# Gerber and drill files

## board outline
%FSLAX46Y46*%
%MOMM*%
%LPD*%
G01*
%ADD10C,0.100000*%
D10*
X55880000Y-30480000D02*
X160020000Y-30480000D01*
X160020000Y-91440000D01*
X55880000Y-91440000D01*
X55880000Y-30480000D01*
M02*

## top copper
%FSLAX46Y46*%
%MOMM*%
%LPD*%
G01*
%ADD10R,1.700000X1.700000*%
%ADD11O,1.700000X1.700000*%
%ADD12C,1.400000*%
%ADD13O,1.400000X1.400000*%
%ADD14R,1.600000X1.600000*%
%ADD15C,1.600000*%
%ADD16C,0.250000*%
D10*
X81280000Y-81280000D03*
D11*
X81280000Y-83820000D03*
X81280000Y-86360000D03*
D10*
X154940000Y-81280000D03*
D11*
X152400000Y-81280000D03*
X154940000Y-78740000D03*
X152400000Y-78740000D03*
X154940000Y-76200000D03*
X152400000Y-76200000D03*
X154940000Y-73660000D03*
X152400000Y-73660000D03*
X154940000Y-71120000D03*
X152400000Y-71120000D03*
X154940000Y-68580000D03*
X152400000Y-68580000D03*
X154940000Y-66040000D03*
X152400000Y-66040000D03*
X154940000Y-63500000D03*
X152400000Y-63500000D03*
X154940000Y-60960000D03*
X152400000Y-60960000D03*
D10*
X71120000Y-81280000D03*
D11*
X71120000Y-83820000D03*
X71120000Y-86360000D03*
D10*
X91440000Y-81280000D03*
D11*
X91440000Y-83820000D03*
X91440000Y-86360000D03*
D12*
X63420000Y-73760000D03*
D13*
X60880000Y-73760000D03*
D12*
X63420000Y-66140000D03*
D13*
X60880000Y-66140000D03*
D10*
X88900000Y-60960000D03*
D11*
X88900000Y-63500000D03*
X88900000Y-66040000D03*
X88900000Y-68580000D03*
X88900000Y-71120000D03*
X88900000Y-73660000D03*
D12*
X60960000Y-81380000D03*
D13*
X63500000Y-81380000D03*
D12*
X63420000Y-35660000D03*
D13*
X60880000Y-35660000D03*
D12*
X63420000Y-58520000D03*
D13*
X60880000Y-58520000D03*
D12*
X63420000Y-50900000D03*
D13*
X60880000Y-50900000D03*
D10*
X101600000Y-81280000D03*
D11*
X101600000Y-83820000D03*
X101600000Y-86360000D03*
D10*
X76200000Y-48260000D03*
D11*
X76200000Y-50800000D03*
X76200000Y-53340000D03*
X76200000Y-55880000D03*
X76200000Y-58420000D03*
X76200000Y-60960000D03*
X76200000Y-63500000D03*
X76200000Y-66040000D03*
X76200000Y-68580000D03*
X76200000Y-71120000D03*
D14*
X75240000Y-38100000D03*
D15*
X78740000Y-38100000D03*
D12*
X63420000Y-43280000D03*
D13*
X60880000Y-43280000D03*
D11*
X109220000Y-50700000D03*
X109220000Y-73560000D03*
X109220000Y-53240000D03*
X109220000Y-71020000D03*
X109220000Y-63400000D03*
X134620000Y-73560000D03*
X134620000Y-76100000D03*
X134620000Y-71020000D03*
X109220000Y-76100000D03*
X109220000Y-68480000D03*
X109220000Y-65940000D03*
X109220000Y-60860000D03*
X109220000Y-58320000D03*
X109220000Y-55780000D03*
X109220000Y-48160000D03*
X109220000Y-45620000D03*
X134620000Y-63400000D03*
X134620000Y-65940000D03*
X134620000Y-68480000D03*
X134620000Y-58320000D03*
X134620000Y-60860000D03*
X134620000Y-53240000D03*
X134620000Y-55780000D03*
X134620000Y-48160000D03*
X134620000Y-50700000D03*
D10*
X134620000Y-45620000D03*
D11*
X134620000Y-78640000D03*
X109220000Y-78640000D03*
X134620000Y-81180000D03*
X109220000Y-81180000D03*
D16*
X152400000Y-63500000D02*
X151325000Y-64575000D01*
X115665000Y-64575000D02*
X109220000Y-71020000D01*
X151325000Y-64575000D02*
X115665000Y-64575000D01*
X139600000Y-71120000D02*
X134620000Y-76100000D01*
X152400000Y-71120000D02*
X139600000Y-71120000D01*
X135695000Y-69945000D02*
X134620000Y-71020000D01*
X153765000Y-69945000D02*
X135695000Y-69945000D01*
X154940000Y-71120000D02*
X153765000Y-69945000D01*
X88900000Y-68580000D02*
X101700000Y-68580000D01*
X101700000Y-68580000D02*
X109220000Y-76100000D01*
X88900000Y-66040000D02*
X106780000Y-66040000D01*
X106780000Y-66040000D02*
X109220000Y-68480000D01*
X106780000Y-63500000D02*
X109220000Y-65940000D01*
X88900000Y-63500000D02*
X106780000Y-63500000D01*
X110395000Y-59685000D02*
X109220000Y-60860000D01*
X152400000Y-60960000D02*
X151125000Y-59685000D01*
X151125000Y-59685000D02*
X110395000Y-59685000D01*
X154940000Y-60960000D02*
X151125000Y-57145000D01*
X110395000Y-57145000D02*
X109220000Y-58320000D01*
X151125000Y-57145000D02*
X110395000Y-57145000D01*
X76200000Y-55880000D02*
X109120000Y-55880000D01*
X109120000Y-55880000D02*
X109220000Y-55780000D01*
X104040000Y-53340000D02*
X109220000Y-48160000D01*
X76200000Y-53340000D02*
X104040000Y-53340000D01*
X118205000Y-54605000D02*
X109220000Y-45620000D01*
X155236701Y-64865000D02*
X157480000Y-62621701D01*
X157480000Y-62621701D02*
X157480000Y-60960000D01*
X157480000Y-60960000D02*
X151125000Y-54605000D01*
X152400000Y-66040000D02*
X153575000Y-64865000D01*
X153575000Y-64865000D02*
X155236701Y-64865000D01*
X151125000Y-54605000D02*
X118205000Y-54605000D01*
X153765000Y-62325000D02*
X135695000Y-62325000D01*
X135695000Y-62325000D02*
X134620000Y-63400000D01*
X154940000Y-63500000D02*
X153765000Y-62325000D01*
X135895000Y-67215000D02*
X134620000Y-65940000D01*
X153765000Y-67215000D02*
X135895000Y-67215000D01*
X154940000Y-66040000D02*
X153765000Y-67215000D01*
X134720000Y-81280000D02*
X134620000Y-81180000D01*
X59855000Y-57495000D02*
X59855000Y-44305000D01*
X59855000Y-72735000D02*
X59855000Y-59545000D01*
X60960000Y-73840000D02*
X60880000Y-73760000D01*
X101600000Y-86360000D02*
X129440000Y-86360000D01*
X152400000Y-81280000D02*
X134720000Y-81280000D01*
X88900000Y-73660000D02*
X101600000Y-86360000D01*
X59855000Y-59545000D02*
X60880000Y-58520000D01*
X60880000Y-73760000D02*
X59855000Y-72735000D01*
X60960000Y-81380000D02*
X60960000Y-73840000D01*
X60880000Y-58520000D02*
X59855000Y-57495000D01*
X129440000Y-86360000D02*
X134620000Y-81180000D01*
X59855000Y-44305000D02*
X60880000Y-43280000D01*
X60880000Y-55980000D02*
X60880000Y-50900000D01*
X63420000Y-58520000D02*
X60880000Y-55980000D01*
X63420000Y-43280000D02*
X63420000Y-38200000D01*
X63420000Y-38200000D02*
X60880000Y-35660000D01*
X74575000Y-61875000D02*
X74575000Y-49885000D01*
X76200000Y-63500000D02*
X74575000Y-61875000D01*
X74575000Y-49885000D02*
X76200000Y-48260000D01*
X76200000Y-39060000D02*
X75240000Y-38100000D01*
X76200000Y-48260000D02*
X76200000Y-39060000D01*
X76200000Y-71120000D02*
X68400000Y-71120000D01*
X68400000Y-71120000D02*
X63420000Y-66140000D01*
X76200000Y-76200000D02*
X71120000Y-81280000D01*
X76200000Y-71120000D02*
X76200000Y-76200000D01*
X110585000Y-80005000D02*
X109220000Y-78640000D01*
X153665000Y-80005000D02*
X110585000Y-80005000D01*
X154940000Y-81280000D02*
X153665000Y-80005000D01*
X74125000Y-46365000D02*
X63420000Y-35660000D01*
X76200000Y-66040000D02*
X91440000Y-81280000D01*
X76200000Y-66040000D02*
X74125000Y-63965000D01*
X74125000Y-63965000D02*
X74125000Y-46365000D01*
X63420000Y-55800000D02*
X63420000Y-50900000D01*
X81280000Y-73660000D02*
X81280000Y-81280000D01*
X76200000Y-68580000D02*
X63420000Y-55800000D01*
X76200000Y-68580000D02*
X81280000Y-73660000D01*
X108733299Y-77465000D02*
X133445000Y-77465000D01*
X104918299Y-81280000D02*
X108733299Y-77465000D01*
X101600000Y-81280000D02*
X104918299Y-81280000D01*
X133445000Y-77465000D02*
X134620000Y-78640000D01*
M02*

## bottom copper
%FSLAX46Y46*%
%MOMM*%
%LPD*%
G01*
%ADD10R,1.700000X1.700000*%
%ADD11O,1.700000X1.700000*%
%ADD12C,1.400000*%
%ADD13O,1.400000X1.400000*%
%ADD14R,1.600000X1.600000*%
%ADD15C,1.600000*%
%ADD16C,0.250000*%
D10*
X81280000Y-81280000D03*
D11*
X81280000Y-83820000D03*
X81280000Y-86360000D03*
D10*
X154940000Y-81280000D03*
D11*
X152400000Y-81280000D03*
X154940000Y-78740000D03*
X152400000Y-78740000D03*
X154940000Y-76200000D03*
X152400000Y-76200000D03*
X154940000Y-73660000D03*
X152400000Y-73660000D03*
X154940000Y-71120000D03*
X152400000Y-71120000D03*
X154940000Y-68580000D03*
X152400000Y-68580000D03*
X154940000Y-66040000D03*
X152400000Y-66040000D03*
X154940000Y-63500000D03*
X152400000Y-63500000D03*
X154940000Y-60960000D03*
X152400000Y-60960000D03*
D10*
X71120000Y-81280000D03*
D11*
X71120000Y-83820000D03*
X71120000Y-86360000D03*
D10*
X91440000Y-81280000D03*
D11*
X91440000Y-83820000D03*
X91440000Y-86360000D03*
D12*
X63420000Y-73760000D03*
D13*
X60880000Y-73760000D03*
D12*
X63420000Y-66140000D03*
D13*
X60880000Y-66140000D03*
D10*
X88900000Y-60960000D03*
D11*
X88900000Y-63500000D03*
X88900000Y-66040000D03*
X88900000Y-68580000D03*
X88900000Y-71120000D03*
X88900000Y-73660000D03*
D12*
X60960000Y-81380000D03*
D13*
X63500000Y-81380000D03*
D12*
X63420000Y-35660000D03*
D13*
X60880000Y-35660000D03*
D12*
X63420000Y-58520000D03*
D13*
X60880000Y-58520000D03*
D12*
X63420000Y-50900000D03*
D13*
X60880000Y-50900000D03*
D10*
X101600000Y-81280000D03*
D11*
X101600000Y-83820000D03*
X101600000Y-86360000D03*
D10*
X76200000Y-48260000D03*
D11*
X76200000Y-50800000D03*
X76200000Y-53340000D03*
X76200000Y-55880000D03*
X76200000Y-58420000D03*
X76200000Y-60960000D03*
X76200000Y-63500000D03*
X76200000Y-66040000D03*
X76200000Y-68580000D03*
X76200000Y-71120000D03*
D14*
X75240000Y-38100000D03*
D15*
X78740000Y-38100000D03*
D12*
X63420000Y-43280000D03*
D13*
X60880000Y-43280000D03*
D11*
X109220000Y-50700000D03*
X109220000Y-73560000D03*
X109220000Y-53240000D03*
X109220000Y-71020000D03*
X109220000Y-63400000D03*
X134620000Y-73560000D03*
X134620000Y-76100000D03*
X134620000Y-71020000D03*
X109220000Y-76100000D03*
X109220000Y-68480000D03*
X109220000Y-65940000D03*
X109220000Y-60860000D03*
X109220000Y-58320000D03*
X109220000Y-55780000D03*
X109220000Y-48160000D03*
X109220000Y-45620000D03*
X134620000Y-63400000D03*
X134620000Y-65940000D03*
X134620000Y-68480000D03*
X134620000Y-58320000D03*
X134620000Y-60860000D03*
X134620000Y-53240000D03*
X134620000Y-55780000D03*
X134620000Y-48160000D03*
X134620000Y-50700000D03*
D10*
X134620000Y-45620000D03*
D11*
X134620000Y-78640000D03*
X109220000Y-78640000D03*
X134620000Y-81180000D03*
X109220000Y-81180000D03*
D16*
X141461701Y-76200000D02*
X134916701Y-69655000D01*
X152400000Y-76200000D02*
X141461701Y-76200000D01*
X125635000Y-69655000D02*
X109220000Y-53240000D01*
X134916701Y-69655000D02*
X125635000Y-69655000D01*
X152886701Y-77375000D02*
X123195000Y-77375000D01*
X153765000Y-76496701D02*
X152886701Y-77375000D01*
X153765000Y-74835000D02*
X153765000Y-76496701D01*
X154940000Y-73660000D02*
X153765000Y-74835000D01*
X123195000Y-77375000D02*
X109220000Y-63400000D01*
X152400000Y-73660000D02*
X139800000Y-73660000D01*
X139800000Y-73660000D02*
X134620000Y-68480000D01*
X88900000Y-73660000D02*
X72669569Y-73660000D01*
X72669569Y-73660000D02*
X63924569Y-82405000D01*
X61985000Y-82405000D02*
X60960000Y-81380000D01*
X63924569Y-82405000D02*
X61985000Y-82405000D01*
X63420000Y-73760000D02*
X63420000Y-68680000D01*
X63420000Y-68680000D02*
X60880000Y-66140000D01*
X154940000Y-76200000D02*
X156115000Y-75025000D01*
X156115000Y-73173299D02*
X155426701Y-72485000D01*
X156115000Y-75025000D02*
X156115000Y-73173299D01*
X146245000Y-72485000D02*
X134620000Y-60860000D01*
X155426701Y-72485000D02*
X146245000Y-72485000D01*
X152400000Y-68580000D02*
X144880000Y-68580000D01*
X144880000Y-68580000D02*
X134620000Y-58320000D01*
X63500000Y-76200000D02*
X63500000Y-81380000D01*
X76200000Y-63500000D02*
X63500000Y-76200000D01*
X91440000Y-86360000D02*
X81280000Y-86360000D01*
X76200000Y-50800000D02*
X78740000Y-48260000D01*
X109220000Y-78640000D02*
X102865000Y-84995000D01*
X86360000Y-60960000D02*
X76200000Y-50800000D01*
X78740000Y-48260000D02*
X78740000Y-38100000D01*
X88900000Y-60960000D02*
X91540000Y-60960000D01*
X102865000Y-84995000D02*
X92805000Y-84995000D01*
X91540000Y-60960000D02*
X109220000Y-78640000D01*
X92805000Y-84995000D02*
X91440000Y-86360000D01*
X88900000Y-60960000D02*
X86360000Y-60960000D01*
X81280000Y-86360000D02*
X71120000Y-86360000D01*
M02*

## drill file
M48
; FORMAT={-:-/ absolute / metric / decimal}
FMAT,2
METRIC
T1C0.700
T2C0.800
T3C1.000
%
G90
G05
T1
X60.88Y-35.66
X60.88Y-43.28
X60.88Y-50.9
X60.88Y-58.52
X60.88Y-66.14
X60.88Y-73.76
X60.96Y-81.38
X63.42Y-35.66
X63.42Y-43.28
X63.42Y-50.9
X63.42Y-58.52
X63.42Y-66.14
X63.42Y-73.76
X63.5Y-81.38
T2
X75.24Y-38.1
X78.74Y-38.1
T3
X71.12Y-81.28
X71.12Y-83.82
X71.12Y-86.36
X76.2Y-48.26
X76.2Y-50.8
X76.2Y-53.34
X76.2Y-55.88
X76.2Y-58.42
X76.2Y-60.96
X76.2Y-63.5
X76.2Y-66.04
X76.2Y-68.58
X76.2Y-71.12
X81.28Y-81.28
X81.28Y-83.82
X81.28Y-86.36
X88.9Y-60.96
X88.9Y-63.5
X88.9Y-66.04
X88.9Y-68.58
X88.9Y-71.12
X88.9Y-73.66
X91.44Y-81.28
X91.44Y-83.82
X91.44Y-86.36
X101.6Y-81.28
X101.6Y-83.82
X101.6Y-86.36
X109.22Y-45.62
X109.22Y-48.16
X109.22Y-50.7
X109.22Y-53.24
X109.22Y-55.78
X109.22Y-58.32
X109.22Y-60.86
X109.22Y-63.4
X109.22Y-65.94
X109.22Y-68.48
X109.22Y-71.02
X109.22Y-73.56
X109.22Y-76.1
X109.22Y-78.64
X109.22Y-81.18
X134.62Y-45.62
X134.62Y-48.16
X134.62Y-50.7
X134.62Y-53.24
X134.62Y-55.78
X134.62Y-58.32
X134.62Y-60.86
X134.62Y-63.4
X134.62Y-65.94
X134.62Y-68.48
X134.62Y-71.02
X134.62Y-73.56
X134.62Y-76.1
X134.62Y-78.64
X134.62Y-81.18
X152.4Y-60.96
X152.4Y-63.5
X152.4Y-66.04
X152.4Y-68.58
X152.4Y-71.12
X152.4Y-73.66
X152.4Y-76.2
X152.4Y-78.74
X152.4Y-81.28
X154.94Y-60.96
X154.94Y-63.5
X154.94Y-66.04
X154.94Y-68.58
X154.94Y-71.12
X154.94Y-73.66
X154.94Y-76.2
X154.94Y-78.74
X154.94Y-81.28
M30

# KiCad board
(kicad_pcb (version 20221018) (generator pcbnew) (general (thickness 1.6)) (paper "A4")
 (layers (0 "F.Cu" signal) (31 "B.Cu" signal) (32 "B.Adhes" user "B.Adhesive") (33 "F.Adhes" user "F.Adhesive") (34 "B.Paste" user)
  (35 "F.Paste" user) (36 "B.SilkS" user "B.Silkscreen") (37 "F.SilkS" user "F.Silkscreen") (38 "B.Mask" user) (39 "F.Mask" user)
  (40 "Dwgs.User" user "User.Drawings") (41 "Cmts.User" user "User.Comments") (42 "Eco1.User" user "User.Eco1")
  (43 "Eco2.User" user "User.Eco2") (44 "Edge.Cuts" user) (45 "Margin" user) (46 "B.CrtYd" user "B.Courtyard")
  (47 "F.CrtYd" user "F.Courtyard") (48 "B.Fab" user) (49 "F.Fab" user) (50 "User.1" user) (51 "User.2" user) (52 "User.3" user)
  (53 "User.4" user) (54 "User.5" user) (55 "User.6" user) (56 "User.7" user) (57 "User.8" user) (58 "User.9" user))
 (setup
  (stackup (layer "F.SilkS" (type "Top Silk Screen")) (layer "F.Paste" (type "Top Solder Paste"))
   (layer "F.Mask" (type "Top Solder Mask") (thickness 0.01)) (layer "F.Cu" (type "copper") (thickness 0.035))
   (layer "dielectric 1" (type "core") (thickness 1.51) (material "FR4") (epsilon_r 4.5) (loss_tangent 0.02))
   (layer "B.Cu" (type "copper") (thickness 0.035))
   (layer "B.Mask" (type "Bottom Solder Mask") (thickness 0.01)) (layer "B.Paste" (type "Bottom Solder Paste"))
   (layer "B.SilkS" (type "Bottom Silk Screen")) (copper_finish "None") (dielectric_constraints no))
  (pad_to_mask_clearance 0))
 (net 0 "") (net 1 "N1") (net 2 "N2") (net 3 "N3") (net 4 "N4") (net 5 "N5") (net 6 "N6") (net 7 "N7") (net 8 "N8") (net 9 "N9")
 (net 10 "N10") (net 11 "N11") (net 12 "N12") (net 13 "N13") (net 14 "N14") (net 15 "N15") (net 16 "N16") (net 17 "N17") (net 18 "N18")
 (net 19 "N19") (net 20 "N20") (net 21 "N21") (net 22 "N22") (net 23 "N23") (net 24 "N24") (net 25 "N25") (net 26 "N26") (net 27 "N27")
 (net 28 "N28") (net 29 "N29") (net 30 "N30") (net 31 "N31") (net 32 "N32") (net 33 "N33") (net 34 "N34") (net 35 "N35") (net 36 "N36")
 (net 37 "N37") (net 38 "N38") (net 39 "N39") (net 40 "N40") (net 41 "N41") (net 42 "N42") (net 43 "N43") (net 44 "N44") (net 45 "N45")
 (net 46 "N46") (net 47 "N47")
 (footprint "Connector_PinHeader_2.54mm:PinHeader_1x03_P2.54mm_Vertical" (layer "F.Cu") (at 81.28 81.28)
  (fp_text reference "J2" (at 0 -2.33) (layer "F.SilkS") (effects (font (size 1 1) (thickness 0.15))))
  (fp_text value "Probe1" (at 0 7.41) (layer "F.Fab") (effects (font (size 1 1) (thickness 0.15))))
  (pad "1" thru_hole rect (at 0 0) (size 1.7 1.7) (drill 1) (layers "*.Cu" "*.Mask") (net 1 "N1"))
  (pad "2" thru_hole oval (at 0 2.54) (size 1.7 1.7) (drill 1) (layers "*.Cu" "*.Mask") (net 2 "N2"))
  (pad "3" thru_hole oval (at 0 5.08) (size 1.7 1.7) (drill 1) (layers "*.Cu" "*.Mask") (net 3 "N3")))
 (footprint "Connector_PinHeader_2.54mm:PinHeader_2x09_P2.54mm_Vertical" (layer "F.Cu") (at 154.94 81.28 180)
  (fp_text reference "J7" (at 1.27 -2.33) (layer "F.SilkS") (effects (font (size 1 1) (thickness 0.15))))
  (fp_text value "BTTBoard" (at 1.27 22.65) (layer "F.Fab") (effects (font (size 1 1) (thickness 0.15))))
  (pad "1" thru_hole rect (at 0 0 180) (size 1.7 1.7) (drill 1) (layers "*.Cu" "*.Mask") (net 3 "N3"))
  (pad "2" thru_hole oval (at 2.54 0 180) (size 1.7 1.7) (drill 1) (layers "*.Cu" "*.Mask") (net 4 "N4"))
  (pad "3" thru_hole oval (at 0 2.54 180) (size 1.7 1.7) (drill 1) (layers "*.Cu" "*.Mask") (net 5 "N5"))
  (pad "4" thru_hole oval (at 2.54 2.54 180) (size 1.7 1.7) (drill 1) (layers "*.Cu" "*.Mask") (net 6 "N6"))
  (pad "5" thru_hole oval (at 0 5.08 180) (size 1.7 1.7) (drill 1) (layers "*.Cu" "*.Mask") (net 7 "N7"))
  (pad "6" thru_hole oval (at 2.54 5.08 180) (size 1.7 1.7) (drill 1) (layers "*.Cu" "*.Mask") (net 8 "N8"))
  (pad "7" thru_hole oval (at 0 7.62 180) (size 1.7 1.7) (drill 1) (layers "*.Cu" "*.Mask") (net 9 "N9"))
  (pad "8" thru_hole oval (at 2.54 7.62 180) (size 1.7 1.7) (drill 1) (layers "*.Cu" "*.Mask") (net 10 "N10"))
  (pad "9" thru_hole oval (at 0 10.16 180) (size 1.7 1.7) (drill 1) (layers "*.Cu" "*.Mask") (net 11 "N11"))
  (pad "10" thru_hole oval (at 2.54 10.16 180) (size 1.7 1.7) (drill 1) (layers "*.Cu" "*.Mask") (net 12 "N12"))
  (pad "11" thru_hole oval (at 0 12.7 180) (size 1.7 1.7) (drill 1) (layers "*.Cu" "*.Mask") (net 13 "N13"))
  (pad "12" thru_hole oval (at 2.54 12.7 180) (size 1.7 1.7) (drill 1) (layers "*.Cu" "*.Mask") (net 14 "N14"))
  (pad "13" thru_hole oval (at 0 15.24 180) (size 1.7 1.7) (drill 1) (layers "*.Cu" "*.Mask") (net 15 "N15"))
  (pad "14" thru_hole oval (at 2.54 15.24 180) (size 1.7 1.7) (drill 1) (layers "*.Cu" "*.Mask") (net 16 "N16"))
  (pad "15" thru_hole oval (at 0 17.78 180) (size 1.7 1.7) (drill 1) (layers "*.Cu" "*.Mask") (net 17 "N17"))
  (pad "16" thru_hole oval (at 2.54 17.78 180) (size 1.7 1.7) (drill 1) (layers "*.Cu" "*.Mask") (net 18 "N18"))
  (pad "17" thru_hole oval (at 0 20.32 180) (size 1.7 1.7) (drill 1) (layers "*.Cu" "*.Mask") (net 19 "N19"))
  (pad "18" thru_hole oval (at 2.54 20.32 180) (size 1.7 1.7) (drill 1) (layers "*.Cu" "*.Mask") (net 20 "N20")))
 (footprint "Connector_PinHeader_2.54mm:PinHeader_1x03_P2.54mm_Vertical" (layer "F.Cu") (at 71.12 81.28)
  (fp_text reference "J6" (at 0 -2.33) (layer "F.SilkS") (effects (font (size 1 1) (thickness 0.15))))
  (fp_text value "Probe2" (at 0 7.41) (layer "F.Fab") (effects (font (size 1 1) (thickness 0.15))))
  (pad "1" thru_hole rect (at 0 0) (size 1.7 1.7) (drill 1) (layers "*.Cu" "*.Mask") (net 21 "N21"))
  (pad "2" thru_hole oval (at 0 2.54) (size 1.7 1.7) (drill 1) (layers "*.Cu" "*.Mask") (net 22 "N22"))
  (pad "3" thru_hole oval (at 0 5.08) (size 1.7 1.7) (drill 1) (layers "*.Cu" "*.Mask") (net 3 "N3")))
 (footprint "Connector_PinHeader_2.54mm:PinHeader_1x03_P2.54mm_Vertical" (layer "F.Cu") (at 91.44 81.28)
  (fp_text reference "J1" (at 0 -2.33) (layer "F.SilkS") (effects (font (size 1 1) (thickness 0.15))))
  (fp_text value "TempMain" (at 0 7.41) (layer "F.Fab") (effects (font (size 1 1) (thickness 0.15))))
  (pad "1" thru_hole rect (at 0 0) (size 1.7 1.7) (drill 1) (layers "*.Cu" "*.Mask") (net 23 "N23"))
  (pad "2" thru_hole oval (at 0 2.54) (size 1.7 1.7) (drill 1) (layers "*.Cu" "*.Mask") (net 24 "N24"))
  (pad "3" thru_hole oval (at 0 5.08) (size 1.7 1.7) (drill 1) (layers "*.Cu" "*.Mask") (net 3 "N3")))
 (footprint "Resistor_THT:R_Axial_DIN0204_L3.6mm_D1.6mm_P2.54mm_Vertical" (layer "F.Cu") (at 63.42 73.76 180)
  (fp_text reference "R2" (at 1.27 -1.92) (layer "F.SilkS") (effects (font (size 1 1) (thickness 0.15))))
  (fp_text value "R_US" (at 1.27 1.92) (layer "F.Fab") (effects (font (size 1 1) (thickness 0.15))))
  (pad "1" thru_hole circle (at 0 0 180) (size 1.4 1.4) (drill 0.7) (layers "*.Cu" "*.Mask") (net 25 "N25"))
  (pad "2" thru_hole oval (at 2.54 0 180) (size 1.4 1.4) (drill 0.7) (layers "*.Cu" "*.Mask") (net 4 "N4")))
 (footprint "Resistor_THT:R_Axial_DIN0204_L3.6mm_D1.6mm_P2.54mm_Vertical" (layer "F.Cu") (at 63.42 66.14 180)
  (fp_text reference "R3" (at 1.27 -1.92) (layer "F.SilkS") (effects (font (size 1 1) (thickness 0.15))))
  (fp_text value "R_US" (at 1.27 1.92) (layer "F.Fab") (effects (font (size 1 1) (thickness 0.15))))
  (pad "1" thru_hole circle (at 0 0 180) (size 1.4 1.4) (drill 0.7) (layers "*.Cu" "*.Mask") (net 21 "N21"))
  (pad "2" thru_hole oval (at 2.54 0 180) (size 1.4 1.4) (drill 0.7) (layers "*.Cu" "*.Mask") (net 25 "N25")))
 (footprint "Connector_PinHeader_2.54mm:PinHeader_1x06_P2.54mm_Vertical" (layer "F.Cu") (at 88.9 60.96)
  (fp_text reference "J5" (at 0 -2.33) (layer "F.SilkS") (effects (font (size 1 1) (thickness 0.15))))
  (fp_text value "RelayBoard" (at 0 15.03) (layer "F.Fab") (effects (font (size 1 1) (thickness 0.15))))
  (pad "1" thru_hole rect (at 0 0) (size 1.7 1.7) (drill 1) (layers "*.Cu" "*.Mask") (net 3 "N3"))
  (pad "2" thru_hole oval (at 0 2.54) (size 1.7 1.7) (drill 1) (layers "*.Cu" "*.Mask") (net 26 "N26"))
  (pad "3" thru_hole oval (at 0 5.08) (size 1.7 1.7) (drill 1) (layers "*.Cu" "*.Mask") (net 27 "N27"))
  (pad "4" thru_hole oval (at 0 7.62) (size 1.7 1.7) (drill 1) (layers "*.Cu" "*.Mask") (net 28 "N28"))
  (pad "5" thru_hole oval (at 0 10.16) (size 1.7 1.7) (drill 1) (layers "*.Cu" "*.Mask") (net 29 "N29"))
  (pad "6" thru_hole oval (at 0 12.7) (size 1.7 1.7) (drill 1) (layers "*.Cu" "*.Mask") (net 4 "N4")))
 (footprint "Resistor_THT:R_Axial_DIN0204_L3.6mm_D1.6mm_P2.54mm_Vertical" (layer "F.Cu") (at 60.96 81.38)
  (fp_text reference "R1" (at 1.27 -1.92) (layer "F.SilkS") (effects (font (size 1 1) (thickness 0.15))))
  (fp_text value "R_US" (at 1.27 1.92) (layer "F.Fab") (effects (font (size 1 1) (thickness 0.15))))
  (pad "1" thru_hole circle (at 0 0) (size 1.4 1.4) (drill 0.7) (layers "*.Cu" "*.Mask") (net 4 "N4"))
  (pad "2" thru_hole oval (at 2.54 0) (size 1.4 1.4) (drill 0.7) (layers "*.Cu" "*.Mask") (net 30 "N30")))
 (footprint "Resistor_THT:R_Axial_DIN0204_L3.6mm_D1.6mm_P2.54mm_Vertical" (layer "F.Cu") (at 63.42 35.66 180)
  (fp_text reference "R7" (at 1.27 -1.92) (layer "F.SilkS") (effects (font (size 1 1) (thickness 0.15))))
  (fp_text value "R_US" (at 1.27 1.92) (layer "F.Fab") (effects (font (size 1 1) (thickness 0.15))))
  (pad "1" thru_hole circle (at 0 0 180) (size 1.4 1.4) (drill 0.7) (layers "*.Cu" "*.Mask") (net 23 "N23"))
  (pad "2" thru_hole oval (at 2.54 0 180) (size 1.4 1.4) (drill 0.7) (layers "*.Cu" "*.Mask") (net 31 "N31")))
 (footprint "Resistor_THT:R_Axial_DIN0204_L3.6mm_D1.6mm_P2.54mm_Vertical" (layer "F.Cu") (at 63.42 58.52 180)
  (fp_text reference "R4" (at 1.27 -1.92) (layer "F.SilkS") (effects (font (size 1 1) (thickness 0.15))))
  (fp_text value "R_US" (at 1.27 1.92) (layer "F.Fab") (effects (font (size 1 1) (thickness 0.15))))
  (pad "1" thru_hole circle (at 0 0 180) (size 1.4 1.4) (drill 0.7) (layers "*.Cu" "*.Mask") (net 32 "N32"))
  (pad "2" thru_hole oval (at 2.54 0 180) (size 1.4 1.4) (drill 0.7) (layers "*.Cu" "*.Mask") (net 4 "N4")))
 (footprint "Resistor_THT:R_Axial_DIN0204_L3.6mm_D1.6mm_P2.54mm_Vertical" (layer "F.Cu") (at 63.42 50.9 180)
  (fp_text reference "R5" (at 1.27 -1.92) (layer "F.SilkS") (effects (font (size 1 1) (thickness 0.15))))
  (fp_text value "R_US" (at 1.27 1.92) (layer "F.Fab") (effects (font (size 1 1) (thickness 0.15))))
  (pad "1" thru_hole circle (at 0 0 180) (size 1.4 1.4) (drill 0.7) (layers "*.Cu" "*.Mask") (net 1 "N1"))
  (pad "2" thru_hole oval (at 2.54 0 180) (size 1.4 1.4) (drill 0.7) (layers "*.Cu" "*.Mask") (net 32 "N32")))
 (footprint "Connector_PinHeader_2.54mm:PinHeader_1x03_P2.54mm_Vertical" (layer "F.Cu") (at 101.6 81.28)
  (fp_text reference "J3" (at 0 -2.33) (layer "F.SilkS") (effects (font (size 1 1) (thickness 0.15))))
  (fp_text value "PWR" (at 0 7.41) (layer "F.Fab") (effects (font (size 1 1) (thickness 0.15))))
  (pad "1" thru_hole rect (at 0 0) (size 1.7 1.7) (drill 1) (layers "*.Cu" "*.Mask") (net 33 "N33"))
  (pad "2" thru_hole oval (at 0 2.54) (size 1.7 1.7) (drill 1) (layers "*.Cu" "*.Mask") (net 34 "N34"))
  (pad "3" thru_hole oval (at 0 5.08) (size 1.7 1.7) (drill 1) (layers "*.Cu" "*.Mask") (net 4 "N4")))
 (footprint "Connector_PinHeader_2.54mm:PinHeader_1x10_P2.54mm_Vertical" (layer "F.Cu") (at 76.2 48.26)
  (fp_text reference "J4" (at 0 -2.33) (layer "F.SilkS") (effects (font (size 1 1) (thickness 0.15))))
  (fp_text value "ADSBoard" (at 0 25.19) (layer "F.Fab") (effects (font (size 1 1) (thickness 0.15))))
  (pad "1" thru_hole rect (at 0 0) (size 1.7 1.7) (drill 1) (layers "*.Cu" "*.Mask") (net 30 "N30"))
  (pad "2" thru_hole oval (at 0 2.54) (size 1.7 1.7) (drill 1) (layers "*.Cu" "*.Mask") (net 3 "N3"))
  (pad "3" thru_hole oval (at 0 5.08) (size 1.7 1.7) (drill 1) (layers "*.Cu" "*.Mask") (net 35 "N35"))
  (pad "4" thru_hole oval (at 0 7.62) (size 1.7 1.7) (drill 1) (layers "*.Cu" "*.Mask") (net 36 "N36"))
  (pad "5" thru_hole oval (at 0 10.16) (size 1.7 1.7) (drill 1) (layers "*.Cu" "*.Mask") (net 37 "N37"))
  (pad "6" thru_hole oval (at 0 12.7) (size 1.7 1.7) (drill 1) (layers "*.Cu" "*.Mask") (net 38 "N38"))
  (pad "7" thru_hole oval (at 0 15.24) (size 1.7 1.7) (drill 1) (layers "*.Cu" "*.Mask") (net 30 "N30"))
  (pad "8" thru_hole oval (at 0 17.78) (size 1.7 1.7) (drill 1) (layers "*.Cu" "*.Mask") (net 23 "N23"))
  (pad "9" thru_hole oval (at 0 20.32) (size 1.7 1.7) (drill 1) (layers "*.Cu" "*.Mask") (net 1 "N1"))
  (pad "10" thru_hole oval (at 0 22.86) (size 1.7 1.7) (drill 1) (layers "*.Cu" "*.Mask") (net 21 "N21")))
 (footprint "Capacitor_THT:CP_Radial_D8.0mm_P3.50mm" (layer "F.Cu") (at 75.24 38.1)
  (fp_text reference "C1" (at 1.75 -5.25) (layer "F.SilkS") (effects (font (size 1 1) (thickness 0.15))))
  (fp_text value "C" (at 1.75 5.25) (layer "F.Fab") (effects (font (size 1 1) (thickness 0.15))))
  (pad "1" thru_hole rect (at 0 0) (size 1.6 1.6) (drill 0.8) (layers "*.Cu" "*.Mask") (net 30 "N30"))
  (pad "2" thru_hole circle (at 3.5 0) (size 1.6 1.6) (drill 0.8) (layers "*.Cu" "*.Mask") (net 3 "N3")))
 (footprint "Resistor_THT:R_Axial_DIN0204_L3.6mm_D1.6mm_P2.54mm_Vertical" (layer "F.Cu") (at 63.42 43.28 180)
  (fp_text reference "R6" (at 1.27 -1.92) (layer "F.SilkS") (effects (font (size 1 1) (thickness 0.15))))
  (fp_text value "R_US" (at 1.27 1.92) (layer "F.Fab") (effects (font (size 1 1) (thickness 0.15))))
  (pad "1" thru_hole circle (at 0 0 180) (size 1.4 1.4) (drill 0.7) (layers "*.Cu" "*.Mask") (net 31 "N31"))
  (pad "2" thru_hole oval (at 2.54 0 180) (size 1.4 1.4) (drill 0.7) (layers "*.Cu" "*.Mask") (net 4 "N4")))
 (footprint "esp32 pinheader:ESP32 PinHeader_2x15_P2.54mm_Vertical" (layer "B.Cu") (at 134.62 45.62 180)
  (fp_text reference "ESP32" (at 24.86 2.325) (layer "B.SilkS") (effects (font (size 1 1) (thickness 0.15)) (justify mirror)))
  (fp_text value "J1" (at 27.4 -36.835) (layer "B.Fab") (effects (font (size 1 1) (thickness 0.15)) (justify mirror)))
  (pad "1" thru_hole oval (at 25.4 -5.08 180) (size 1.7 1.7) (drill 1) (layers "*.Cu" "*.Mask") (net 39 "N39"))
  (pad "2" thru_hole oval (at 25.4 -27.94 180) (size 1.7 1.7) (drill 1) (layers "*.Cu" "*.Mask") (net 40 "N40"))
  (pad "3" thru_hole oval (at 25.4 -7.62 180) (size 1.7 1.7) (drill 1) (layers "*.Cu" "*.Mask") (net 8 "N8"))
  (pad "4" thru_hole oval (at 25.4 -25.4 180) (size 1.7 1.7) (drill 1) (layers "*.Cu" "*.Mask") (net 18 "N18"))
  (pad "5" thru_hole oval (at 25.4 -17.78 180) (size 1.7 1.7) (drill 1) (layers "*.Cu" "*.Mask") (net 9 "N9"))
  (pad "12" thru_hole oval (at 0 -27.94 180) (size 1.7 1.7) (drill 1) (layers "*.Cu" "*.Mask") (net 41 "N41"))
  (pad "13" thru_hole oval (at 0 -30.48 180) (size 1.7 1.7) (drill 1) (layers "*.Cu" "*.Mask") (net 12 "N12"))
  (pad "14" thru_hole oval (at 0 -25.4 180) (size 1.7 1.7) (drill 1) (layers "*.Cu" "*.Mask") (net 11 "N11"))
  (pad "15" thru_hole oval (at 25.4 -30.48 180) (size 1.7 1.7) (drill 1) (layers "*.Cu" "*.Mask") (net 28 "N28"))
  (pad "16" thru_hole oval (at 25.4 -22.86 180) (size 1.7 1.7) (drill 1) (layers "*.Cu" "*.Mask") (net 27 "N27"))
  (pad "17" thru_hole oval (at 25.4 -20.32 180) (size 1.7 1.7) (drill 1) (layers "*.Cu" "*.Mask") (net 26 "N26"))
  (pad "18" thru_hole oval (at 25.4 -15.24 180) (size 1.7 1.7) (drill 1) (layers "*.Cu" "*.Mask") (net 20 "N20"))
  (pad "19" thru_hole oval (at 25.4 -12.7 180) (size 1.7 1.7) (drill 1) (layers "*.Cu" "*.Mask") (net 19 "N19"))
  (pad "21" thru_hole oval (at 25.4 -10.16 180) (size 1.7 1.7) (drill 1) (layers "*.Cu" "*.Mask") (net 36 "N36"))
  (pad "22" thru_hole oval (at 25.4 -2.54 180) (size 1.7 1.7) (drill 1) (layers "*.Cu" "*.Mask") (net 35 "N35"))
  (pad "23" thru_hole oval (at 25.4 0 180) (size 1.7 1.7) (drill 1) (layers "*.Cu" "*.Mask") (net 16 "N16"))
  (pad "25" thru_hole oval (at 0 -17.78 180) (size 1.7 1.7) (drill 1) (layers "*.Cu" "*.Mask") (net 17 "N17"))
  (pad "26" thru_hole oval (at 0 -20.32 180) (size 1.7 1.7) (drill 1) (layers "*.Cu" "*.Mask") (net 15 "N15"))
  (pad "27" thru_hole oval (at 0 -22.86 180) (size 1.7 1.7) (drill 1) (layers "*.Cu" "*.Mask") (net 10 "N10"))
  (pad "32" thru_hole oval (at 0 -12.7 180) (size 1.7 1.7) (drill 1) (layers "*.Cu" "*.Mask") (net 14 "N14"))
  (pad "33" thru_hole oval (at 0 -15.24 180) (size 1.7 1.7) (drill 1) (layers "*.Cu" "*.Mask") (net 7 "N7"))
  (pad "34" thru_hole oval (at 0 -7.62 180) (size 1.7 1.7) (drill 1) (layers "*.Cu" "*.Mask") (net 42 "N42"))
  (pad "35" thru_hole oval (at 0 -10.16 180) (size 1.7 1.7) (drill 1) (layers "*.Cu" "*.Mask") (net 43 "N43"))
  (pad "36" thru_hole oval (at 0 -2.54 180) (size 1.7 1.7) (drill 1) (layers "*.Cu" "*.Mask") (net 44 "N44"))
  (pad "39" thru_hole oval (at 0 -5.08 180) (size 1.7 1.7) (drill 1) (layers "*.Cu" "*.Mask") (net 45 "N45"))
  (pad "60" thru_hole rect (at 0 0 180) (size 1.7 1.7) (drill 1) (layers "*.Cu" "*.Mask") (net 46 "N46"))
  (pad "61" thru_hole oval (at 0 -33.02 180) (size 1.7 1.7) (drill 1) (layers "*.Cu" "*.Mask") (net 33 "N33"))
  (pad "62" thru_hole oval (at 25.4 -33.02 180) (size 1.7 1.7) (drill 1) (layers "*.Cu" "*.Mask") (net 3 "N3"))
  (pad "63" thru_hole oval (at 0 -35.56 180) (size 1.7 1.7) (drill 1) (layers "*.Cu" "*.Mask") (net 4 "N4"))
  (pad "64" thru_hole oval (at 25.4 -35.56 180) (size 1.7 1.7) (drill 1) (layers "*.Cu" "*.Mask") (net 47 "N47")))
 (gr_rect (start 55.88 30.48) (end 160.02 91.44) (stroke (width 0.1) (type default)) (fill none) (layer "Edge.Cuts"))
 (segment (start 141.461701 76.2) (end 134.916701 69.655) (width 0.25) (layer "B.Cu") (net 8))
 (segment (start 152.4 76.2) (end 141.461701 76.2) (width 0.25) (layer "B.Cu") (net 8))
 (segment (start 125.635 69.655) (end 109.22 53.24) (width 0.25) (layer "B.Cu") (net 8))
 (segment (start 134.916701 69.655) (end 125.635 69.655) (width 0.25) (layer "B.Cu") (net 8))
 (segment (start 152.4 63.5) (end 151.325 64.575) (width 0.25) (layer "F.Cu") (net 18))
 (segment (start 115.665 64.575) (end 109.22 71.02) (width 0.25) (layer "F.Cu") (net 18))
 (segment (start 151.325 64.575) (end 115.665 64.575) (width 0.25) (layer "F.Cu") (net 18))
 (segment (start 152.886701 77.375) (end 123.195 77.375) (width 0.25) (layer "B.Cu") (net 9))
 (segment (start 153.765 76.496701) (end 152.886701 77.375) (width 0.25) (layer "B.Cu") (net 9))
 (segment (start 153.765 74.835) (end 153.765 76.496701) (width 0.25) (layer "B.Cu") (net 9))
 (segment (start 154.94 73.66) (end 153.765 74.835) (width 0.25) (layer "B.Cu") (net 9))
 (segment (start 123.195 77.375) (end 109.22 63.4) (width 0.25) (layer "B.Cu") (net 9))
 (segment (start 139.6 71.12) (end 134.62 76.1) (width 0.25) (layer "F.Cu") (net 12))
 (segment (start 152.4 71.12) (end 139.6 71.12) (width 0.25) (layer "F.Cu") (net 12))
 (segment (start 135.695 69.945) (end 134.62 71.02) (width 0.25) (layer "F.Cu") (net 11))
 (segment (start 153.765 69.945) (end 135.695 69.945) (width 0.25) (layer "F.Cu") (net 11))
 (segment (start 154.94 71.12) (end 153.765 69.945) (width 0.25) (layer "F.Cu") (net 11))
 (segment (start 88.9 68.58) (end 101.7 68.58) (width 0.25) (layer "F.Cu") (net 28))
 (segment (start 101.7 68.58) (end 109.22 76.1) (width 0.25) (layer "F.Cu") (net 28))
 (segment (start 88.9 66.04) (end 106.78 66.04) (width 0.25) (layer "F.Cu") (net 27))
 (segment (start 106.78 66.04) (end 109.22 68.48) (width 0.25) (layer "F.Cu") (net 27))
 (segment (start 106.78 63.5) (end 109.22 65.94) (width 0.25) (layer "F.Cu") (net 26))
 (segment (start 88.9 63.5) (end 106.78 63.5) (width 0.25) (layer "F.Cu") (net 26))
 (segment (start 110.395 59.685) (end 109.22 60.86) (width 0.25) (layer "F.Cu") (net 20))
 (segment (start 152.4 60.96) (end 151.125 59.685) (width 0.25) (layer "F.Cu") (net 20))
 (segment (start 151.125 59.685) (end 110.395 59.685) (width 0.25) (layer "F.Cu") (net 20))
 (segment (start 154.94 60.96) (end 151.125 57.145) (width 0.25) (layer "F.Cu") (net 19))
 (segment (start 110.395 57.145) (end 109.22 58.32) (width 0.25) (layer "F.Cu") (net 19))
 (segment (start 151.125 57.145) (end 110.395 57.145) (width 0.25) (layer "F.Cu") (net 19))
 (segment (start 76.2 55.88) (end 109.12 55.88) (width 0.25) (layer "F.Cu") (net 36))
 (segment (start 109.12 55.88) (end 109.22 55.78) (width 0.25) (layer "F.Cu") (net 36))
 (segment (start 104.04 53.34) (end 109.22 48.16) (width 0.25) (layer "F.Cu") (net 35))
 (segment (start 76.2 53.34) (end 104.04 53.34) (width 0.25) (layer "F.Cu") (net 35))
 (segment (start 118.205 54.605) (end 109.22 45.62) (width 0.25) (layer "F.Cu") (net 16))
 (segment (start 155.236701 64.865) (end 157.48 62.621701) (width 0.25) (layer "F.Cu") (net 16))
 (segment (start 157.48 62.621701) (end 157.48 60.96) (width 0.25) (layer "F.Cu") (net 16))
 (segment (start 157.48 60.96) (end 151.125 54.605) (width 0.25) (layer "F.Cu") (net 16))
 (segment (start 152.4 66.04) (end 153.575 64.865) (width 0.25) (layer "F.Cu") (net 16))
 (segment (start 153.575 64.865) (end 155.236701 64.865) (width 0.25) (layer "F.Cu") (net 16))
 (segment (start 151.125 54.605) (end 118.205 54.605) (width 0.25) (layer "F.Cu") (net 16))
 (segment (start 153.765 62.325) (end 135.695 62.325) (width 0.25) (layer "F.Cu") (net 17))
 (segment (start 135.695 62.325) (end 134.62 63.4) (width 0.25) (layer "F.Cu") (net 17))
 (segment (start 154.94 63.5) (end 153.765 62.325) (width 0.25) (layer "F.Cu") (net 17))
 (segment (start 135.895 67.215) (end 134.62 65.94) (width 0.25) (layer "F.Cu") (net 15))
 (segment (start 153.765 67.215) (end 135.895 67.215) (width 0.25) (layer "F.Cu") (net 15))
 (segment (start 154.94 66.04) (end 153.765 67.215) (width 0.25) (layer "F.Cu") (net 15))
 (segment (start 152.4 73.66) (end 139.8 73.66) (width 0.25) (layer "B.Cu") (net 10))
 (segment (start 139.8 73.66) (end 134.62 68.48) (width 0.25) (layer "B.Cu") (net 10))
 (segment (start 134.72 81.28) (end 134.62 81.18) (width 0.25) (layer "F.Cu") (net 4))
 (segment (start 59.855 57.495) (end 59.855 44.305) (width 0.25) (layer "F.Cu") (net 4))
 (segment (start 59.855 72.735) (end 59.855 59.545) (width 0.25) (layer "F.Cu") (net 4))
 (segment (start 60.96 73.84) (end 60.88 73.76) (width 0.25) (layer "F.Cu") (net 4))
 (segment (start 101.6 86.36) (end 129.44 86.36) (width 0.25) (layer "F.Cu") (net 4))
 (segment (start 152.4 81.28) (end 134.72 81.28) (width 0.25) (layer "F.Cu") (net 4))
 (segment (start 88.9 73.66) (end 101.6 86.36) (width 0.25) (layer "F.Cu") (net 4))
 (segment (start 59.855 59.545) (end 60.88 58.52) (width 0.25) (layer "F.Cu") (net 4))
 (segment (start 60.88 73.76) (end 59.855 72.735) (width 0.25) (layer "F.Cu") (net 4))
 (segment (start 60.96 81.38) (end 60.96 73.84) (width 0.25) (layer "F.Cu") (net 4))
 (segment (start 60.88 58.52) (end 59.855 57.495) (width 0.25) (layer "F.Cu") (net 4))
 (segment (start 129.44 86.36) (end 134.62 81.18) (width 0.25) (layer "F.Cu") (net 4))
 (segment (start 59.855 44.305) (end 60.88 43.28) (width 0.25) (layer "F.Cu") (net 4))
 (segment (start 88.9 73.66) (end 72.669569 73.66) (width 0.25) (layer "B.Cu") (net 4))
 (segment (start 72.669569 73.66) (end 63.924569 82.405) (width 0.25) (layer "B.Cu") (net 4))
 (segment (start 61.985 82.405) (end 60.96 81.38) (width 0.25) (layer "B.Cu") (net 4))
 (segment (start 63.924569 82.405) (end 61.985 82.405) (width 0.25) (layer "B.Cu") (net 4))
 (segment (start 63.42 73.76) (end 63.42 68.68) (width 0.25) (layer "B.Cu") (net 25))
 (segment (start 63.42 68.68) (end 60.88 66.14) (width 0.25) (layer "B.Cu") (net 25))
 (segment (start 60.88 55.98) (end 60.88 50.9) (width 0.25) (layer "F.Cu") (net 32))
 (segment (start 63.42 58.52) (end 60.88 55.98) (width 0.25) (layer "F.Cu") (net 32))
 (segment (start 63.42 43.28) (end 63.42 38.2) (width 0.25) (layer "F.Cu") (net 31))
 (segment (start 63.42 38.2) (end 60.88 35.66) (width 0.25) (layer "F.Cu") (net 31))
 (segment (start 154.94 76.2) (end 156.115 75.025) (width 0.25) (layer "B.Cu") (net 7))
 (segment (start 156.115 73.173299) (end 155.426701 72.485) (width 0.25) (layer "B.Cu") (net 7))
 (segment (start 156.115 75.025) (end 156.115 73.173299) (width 0.25) (layer "B.Cu") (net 7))
 (segment (start 146.245 72.485) (end 134.62 60.86) (width 0.25) (layer "B.Cu") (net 7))
 (segment (start 155.426701 72.485) (end 146.245 72.485) (width 0.25) (layer "B.Cu") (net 7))
 (segment (start 152.4 68.58) (end 144.88 68.58) (width 0.25) (layer "B.Cu") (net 14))
 (segment (start 144.88 68.58) (end 134.62 58.32) (width 0.25) (layer "B.Cu") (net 14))
 (segment (start 74.575 61.875) (end 74.575 49.885) (width 0.25) (layer "F.Cu") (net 30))
 (segment (start 76.2 63.5) (end 74.575 61.875) (width 0.25) (layer "F.Cu") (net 30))
 (segment (start 74.575 49.885) (end 76.2 48.26) (width 0.25) (layer "F.Cu") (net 30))
 (segment (start 76.2 39.06) (end 75.24 38.1) (width 0.25) (layer "F.Cu") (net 30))
 (segment (start 76.2 48.26) (end 76.2 39.06) (width 0.25) (layer "F.Cu") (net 30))
 (segment (start 63.5 76.2) (end 63.5 81.38) (width 0.25) (layer "B.Cu") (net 30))
 (segment (start 76.2 63.5) (end 63.5 76.2) (width 0.25) (layer "B.Cu") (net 30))
 (segment (start 76.2 71.12) (end 68.4 71.12) (width 0.25) (layer "F.Cu") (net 21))
 (segment (start 68.4 71.12) (end 63.42 66.14) (width 0.25) (layer "F.Cu") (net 21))
 (segment (start 76.2 76.2) (end 71.12 81.28) (width 0.25) (layer "F.Cu") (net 21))
 (segment (start 76.2 71.12) (end 76.2 76.2) (width 0.25) (layer "F.Cu") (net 21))
 (segment (start 110.585 80.005) (end 109.22 78.64) (width 0.25) (layer "F.Cu") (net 3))
 (segment (start 153.665 80.005) (end 110.585 80.005) (width 0.25) (layer "F.Cu") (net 3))
 (segment (start 154.94 81.28) (end 153.665 80.005) (width 0.25) (layer "F.Cu") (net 3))
 (segment (start 91.44 86.36) (end 81.28 86.36) (width 0.25) (layer "B.Cu") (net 3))
 (segment (start 76.2 50.8) (end 78.74 48.26) (width 0.25) (layer "B.Cu") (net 3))
 (segment (start 109.22 78.64) (end 102.865 84.995) (width 0.25) (layer "B.Cu") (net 3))
 (segment (start 86.36 60.96) (end 76.2 50.8) (width 0.25) (layer "B.Cu") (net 3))
 (segment (start 78.74 48.26) (end 78.74 38.1) (width 0.25) (layer "B.Cu") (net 3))
 (segment (start 88.9 60.96) (end 91.54 60.96) (width 0.25) (layer "B.Cu") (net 3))
 (segment (start 102.865 84.995) (end 92.805 84.995) (width 0.25) (layer "B.Cu") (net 3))
 (segment (start 91.54 60.96) (end 109.22 78.64) (width 0.25) (layer "B.Cu") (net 3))
 (segment (start 92.805 84.995) (end 91.44 86.36) (width 0.25) (layer "B.Cu") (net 3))
 (segment (start 88.9 60.96) (end 86.36 60.96) (width 0.25) (layer "B.Cu") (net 3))
 (segment (start 81.28 86.36) (end 71.12 86.36) (width 0.25) (layer "B.Cu") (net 3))
 (segment (start 74.125 46.365) (end 63.42 35.66) (width 0.25) (layer "F.Cu") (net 23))
 (segment (start 76.2 66.04) (end 91.44 81.28) (width 0.25) (layer "F.Cu") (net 23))
 (segment (start 76.2 66.04) (end 74.125 63.965) (width 0.25) (layer "F.Cu") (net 23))
 (segment (start 74.125 63.965) (end 74.125 46.365) (width 0.25) (layer "F.Cu") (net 23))
 (segment (start 63.42 55.8) (end 63.42 50.9) (width 0.25) (layer "F.Cu") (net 1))
 (segment (start 81.28 73.66) (end 81.28 81.28) (width 0.25) (layer "F.Cu") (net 1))
 (segment (start 76.2 68.58) (end 63.42 55.8) (width 0.25) (layer "F.Cu") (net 1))
 (segment (start 76.2 68.58) (end 81.28 73.66) (width 0.25) (layer "F.Cu") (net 1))
 (segment (start 108.733299 77.465) (end 133.445 77.465) (width 0.25) (layer "F.Cu") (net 33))
 (segment (start 104.918299 81.28) (end 108.733299 77.465) (width 0.25) (layer "F.Cu") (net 33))
 (segment (start 101.6 81.28) (end 104.918299 81.28) (width 0.25) (layer "F.Cu") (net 33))
 (segment (start 133.445 77.465) (end 134.62 78.64) (width 0.25) (layer "F.Cu") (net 33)))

